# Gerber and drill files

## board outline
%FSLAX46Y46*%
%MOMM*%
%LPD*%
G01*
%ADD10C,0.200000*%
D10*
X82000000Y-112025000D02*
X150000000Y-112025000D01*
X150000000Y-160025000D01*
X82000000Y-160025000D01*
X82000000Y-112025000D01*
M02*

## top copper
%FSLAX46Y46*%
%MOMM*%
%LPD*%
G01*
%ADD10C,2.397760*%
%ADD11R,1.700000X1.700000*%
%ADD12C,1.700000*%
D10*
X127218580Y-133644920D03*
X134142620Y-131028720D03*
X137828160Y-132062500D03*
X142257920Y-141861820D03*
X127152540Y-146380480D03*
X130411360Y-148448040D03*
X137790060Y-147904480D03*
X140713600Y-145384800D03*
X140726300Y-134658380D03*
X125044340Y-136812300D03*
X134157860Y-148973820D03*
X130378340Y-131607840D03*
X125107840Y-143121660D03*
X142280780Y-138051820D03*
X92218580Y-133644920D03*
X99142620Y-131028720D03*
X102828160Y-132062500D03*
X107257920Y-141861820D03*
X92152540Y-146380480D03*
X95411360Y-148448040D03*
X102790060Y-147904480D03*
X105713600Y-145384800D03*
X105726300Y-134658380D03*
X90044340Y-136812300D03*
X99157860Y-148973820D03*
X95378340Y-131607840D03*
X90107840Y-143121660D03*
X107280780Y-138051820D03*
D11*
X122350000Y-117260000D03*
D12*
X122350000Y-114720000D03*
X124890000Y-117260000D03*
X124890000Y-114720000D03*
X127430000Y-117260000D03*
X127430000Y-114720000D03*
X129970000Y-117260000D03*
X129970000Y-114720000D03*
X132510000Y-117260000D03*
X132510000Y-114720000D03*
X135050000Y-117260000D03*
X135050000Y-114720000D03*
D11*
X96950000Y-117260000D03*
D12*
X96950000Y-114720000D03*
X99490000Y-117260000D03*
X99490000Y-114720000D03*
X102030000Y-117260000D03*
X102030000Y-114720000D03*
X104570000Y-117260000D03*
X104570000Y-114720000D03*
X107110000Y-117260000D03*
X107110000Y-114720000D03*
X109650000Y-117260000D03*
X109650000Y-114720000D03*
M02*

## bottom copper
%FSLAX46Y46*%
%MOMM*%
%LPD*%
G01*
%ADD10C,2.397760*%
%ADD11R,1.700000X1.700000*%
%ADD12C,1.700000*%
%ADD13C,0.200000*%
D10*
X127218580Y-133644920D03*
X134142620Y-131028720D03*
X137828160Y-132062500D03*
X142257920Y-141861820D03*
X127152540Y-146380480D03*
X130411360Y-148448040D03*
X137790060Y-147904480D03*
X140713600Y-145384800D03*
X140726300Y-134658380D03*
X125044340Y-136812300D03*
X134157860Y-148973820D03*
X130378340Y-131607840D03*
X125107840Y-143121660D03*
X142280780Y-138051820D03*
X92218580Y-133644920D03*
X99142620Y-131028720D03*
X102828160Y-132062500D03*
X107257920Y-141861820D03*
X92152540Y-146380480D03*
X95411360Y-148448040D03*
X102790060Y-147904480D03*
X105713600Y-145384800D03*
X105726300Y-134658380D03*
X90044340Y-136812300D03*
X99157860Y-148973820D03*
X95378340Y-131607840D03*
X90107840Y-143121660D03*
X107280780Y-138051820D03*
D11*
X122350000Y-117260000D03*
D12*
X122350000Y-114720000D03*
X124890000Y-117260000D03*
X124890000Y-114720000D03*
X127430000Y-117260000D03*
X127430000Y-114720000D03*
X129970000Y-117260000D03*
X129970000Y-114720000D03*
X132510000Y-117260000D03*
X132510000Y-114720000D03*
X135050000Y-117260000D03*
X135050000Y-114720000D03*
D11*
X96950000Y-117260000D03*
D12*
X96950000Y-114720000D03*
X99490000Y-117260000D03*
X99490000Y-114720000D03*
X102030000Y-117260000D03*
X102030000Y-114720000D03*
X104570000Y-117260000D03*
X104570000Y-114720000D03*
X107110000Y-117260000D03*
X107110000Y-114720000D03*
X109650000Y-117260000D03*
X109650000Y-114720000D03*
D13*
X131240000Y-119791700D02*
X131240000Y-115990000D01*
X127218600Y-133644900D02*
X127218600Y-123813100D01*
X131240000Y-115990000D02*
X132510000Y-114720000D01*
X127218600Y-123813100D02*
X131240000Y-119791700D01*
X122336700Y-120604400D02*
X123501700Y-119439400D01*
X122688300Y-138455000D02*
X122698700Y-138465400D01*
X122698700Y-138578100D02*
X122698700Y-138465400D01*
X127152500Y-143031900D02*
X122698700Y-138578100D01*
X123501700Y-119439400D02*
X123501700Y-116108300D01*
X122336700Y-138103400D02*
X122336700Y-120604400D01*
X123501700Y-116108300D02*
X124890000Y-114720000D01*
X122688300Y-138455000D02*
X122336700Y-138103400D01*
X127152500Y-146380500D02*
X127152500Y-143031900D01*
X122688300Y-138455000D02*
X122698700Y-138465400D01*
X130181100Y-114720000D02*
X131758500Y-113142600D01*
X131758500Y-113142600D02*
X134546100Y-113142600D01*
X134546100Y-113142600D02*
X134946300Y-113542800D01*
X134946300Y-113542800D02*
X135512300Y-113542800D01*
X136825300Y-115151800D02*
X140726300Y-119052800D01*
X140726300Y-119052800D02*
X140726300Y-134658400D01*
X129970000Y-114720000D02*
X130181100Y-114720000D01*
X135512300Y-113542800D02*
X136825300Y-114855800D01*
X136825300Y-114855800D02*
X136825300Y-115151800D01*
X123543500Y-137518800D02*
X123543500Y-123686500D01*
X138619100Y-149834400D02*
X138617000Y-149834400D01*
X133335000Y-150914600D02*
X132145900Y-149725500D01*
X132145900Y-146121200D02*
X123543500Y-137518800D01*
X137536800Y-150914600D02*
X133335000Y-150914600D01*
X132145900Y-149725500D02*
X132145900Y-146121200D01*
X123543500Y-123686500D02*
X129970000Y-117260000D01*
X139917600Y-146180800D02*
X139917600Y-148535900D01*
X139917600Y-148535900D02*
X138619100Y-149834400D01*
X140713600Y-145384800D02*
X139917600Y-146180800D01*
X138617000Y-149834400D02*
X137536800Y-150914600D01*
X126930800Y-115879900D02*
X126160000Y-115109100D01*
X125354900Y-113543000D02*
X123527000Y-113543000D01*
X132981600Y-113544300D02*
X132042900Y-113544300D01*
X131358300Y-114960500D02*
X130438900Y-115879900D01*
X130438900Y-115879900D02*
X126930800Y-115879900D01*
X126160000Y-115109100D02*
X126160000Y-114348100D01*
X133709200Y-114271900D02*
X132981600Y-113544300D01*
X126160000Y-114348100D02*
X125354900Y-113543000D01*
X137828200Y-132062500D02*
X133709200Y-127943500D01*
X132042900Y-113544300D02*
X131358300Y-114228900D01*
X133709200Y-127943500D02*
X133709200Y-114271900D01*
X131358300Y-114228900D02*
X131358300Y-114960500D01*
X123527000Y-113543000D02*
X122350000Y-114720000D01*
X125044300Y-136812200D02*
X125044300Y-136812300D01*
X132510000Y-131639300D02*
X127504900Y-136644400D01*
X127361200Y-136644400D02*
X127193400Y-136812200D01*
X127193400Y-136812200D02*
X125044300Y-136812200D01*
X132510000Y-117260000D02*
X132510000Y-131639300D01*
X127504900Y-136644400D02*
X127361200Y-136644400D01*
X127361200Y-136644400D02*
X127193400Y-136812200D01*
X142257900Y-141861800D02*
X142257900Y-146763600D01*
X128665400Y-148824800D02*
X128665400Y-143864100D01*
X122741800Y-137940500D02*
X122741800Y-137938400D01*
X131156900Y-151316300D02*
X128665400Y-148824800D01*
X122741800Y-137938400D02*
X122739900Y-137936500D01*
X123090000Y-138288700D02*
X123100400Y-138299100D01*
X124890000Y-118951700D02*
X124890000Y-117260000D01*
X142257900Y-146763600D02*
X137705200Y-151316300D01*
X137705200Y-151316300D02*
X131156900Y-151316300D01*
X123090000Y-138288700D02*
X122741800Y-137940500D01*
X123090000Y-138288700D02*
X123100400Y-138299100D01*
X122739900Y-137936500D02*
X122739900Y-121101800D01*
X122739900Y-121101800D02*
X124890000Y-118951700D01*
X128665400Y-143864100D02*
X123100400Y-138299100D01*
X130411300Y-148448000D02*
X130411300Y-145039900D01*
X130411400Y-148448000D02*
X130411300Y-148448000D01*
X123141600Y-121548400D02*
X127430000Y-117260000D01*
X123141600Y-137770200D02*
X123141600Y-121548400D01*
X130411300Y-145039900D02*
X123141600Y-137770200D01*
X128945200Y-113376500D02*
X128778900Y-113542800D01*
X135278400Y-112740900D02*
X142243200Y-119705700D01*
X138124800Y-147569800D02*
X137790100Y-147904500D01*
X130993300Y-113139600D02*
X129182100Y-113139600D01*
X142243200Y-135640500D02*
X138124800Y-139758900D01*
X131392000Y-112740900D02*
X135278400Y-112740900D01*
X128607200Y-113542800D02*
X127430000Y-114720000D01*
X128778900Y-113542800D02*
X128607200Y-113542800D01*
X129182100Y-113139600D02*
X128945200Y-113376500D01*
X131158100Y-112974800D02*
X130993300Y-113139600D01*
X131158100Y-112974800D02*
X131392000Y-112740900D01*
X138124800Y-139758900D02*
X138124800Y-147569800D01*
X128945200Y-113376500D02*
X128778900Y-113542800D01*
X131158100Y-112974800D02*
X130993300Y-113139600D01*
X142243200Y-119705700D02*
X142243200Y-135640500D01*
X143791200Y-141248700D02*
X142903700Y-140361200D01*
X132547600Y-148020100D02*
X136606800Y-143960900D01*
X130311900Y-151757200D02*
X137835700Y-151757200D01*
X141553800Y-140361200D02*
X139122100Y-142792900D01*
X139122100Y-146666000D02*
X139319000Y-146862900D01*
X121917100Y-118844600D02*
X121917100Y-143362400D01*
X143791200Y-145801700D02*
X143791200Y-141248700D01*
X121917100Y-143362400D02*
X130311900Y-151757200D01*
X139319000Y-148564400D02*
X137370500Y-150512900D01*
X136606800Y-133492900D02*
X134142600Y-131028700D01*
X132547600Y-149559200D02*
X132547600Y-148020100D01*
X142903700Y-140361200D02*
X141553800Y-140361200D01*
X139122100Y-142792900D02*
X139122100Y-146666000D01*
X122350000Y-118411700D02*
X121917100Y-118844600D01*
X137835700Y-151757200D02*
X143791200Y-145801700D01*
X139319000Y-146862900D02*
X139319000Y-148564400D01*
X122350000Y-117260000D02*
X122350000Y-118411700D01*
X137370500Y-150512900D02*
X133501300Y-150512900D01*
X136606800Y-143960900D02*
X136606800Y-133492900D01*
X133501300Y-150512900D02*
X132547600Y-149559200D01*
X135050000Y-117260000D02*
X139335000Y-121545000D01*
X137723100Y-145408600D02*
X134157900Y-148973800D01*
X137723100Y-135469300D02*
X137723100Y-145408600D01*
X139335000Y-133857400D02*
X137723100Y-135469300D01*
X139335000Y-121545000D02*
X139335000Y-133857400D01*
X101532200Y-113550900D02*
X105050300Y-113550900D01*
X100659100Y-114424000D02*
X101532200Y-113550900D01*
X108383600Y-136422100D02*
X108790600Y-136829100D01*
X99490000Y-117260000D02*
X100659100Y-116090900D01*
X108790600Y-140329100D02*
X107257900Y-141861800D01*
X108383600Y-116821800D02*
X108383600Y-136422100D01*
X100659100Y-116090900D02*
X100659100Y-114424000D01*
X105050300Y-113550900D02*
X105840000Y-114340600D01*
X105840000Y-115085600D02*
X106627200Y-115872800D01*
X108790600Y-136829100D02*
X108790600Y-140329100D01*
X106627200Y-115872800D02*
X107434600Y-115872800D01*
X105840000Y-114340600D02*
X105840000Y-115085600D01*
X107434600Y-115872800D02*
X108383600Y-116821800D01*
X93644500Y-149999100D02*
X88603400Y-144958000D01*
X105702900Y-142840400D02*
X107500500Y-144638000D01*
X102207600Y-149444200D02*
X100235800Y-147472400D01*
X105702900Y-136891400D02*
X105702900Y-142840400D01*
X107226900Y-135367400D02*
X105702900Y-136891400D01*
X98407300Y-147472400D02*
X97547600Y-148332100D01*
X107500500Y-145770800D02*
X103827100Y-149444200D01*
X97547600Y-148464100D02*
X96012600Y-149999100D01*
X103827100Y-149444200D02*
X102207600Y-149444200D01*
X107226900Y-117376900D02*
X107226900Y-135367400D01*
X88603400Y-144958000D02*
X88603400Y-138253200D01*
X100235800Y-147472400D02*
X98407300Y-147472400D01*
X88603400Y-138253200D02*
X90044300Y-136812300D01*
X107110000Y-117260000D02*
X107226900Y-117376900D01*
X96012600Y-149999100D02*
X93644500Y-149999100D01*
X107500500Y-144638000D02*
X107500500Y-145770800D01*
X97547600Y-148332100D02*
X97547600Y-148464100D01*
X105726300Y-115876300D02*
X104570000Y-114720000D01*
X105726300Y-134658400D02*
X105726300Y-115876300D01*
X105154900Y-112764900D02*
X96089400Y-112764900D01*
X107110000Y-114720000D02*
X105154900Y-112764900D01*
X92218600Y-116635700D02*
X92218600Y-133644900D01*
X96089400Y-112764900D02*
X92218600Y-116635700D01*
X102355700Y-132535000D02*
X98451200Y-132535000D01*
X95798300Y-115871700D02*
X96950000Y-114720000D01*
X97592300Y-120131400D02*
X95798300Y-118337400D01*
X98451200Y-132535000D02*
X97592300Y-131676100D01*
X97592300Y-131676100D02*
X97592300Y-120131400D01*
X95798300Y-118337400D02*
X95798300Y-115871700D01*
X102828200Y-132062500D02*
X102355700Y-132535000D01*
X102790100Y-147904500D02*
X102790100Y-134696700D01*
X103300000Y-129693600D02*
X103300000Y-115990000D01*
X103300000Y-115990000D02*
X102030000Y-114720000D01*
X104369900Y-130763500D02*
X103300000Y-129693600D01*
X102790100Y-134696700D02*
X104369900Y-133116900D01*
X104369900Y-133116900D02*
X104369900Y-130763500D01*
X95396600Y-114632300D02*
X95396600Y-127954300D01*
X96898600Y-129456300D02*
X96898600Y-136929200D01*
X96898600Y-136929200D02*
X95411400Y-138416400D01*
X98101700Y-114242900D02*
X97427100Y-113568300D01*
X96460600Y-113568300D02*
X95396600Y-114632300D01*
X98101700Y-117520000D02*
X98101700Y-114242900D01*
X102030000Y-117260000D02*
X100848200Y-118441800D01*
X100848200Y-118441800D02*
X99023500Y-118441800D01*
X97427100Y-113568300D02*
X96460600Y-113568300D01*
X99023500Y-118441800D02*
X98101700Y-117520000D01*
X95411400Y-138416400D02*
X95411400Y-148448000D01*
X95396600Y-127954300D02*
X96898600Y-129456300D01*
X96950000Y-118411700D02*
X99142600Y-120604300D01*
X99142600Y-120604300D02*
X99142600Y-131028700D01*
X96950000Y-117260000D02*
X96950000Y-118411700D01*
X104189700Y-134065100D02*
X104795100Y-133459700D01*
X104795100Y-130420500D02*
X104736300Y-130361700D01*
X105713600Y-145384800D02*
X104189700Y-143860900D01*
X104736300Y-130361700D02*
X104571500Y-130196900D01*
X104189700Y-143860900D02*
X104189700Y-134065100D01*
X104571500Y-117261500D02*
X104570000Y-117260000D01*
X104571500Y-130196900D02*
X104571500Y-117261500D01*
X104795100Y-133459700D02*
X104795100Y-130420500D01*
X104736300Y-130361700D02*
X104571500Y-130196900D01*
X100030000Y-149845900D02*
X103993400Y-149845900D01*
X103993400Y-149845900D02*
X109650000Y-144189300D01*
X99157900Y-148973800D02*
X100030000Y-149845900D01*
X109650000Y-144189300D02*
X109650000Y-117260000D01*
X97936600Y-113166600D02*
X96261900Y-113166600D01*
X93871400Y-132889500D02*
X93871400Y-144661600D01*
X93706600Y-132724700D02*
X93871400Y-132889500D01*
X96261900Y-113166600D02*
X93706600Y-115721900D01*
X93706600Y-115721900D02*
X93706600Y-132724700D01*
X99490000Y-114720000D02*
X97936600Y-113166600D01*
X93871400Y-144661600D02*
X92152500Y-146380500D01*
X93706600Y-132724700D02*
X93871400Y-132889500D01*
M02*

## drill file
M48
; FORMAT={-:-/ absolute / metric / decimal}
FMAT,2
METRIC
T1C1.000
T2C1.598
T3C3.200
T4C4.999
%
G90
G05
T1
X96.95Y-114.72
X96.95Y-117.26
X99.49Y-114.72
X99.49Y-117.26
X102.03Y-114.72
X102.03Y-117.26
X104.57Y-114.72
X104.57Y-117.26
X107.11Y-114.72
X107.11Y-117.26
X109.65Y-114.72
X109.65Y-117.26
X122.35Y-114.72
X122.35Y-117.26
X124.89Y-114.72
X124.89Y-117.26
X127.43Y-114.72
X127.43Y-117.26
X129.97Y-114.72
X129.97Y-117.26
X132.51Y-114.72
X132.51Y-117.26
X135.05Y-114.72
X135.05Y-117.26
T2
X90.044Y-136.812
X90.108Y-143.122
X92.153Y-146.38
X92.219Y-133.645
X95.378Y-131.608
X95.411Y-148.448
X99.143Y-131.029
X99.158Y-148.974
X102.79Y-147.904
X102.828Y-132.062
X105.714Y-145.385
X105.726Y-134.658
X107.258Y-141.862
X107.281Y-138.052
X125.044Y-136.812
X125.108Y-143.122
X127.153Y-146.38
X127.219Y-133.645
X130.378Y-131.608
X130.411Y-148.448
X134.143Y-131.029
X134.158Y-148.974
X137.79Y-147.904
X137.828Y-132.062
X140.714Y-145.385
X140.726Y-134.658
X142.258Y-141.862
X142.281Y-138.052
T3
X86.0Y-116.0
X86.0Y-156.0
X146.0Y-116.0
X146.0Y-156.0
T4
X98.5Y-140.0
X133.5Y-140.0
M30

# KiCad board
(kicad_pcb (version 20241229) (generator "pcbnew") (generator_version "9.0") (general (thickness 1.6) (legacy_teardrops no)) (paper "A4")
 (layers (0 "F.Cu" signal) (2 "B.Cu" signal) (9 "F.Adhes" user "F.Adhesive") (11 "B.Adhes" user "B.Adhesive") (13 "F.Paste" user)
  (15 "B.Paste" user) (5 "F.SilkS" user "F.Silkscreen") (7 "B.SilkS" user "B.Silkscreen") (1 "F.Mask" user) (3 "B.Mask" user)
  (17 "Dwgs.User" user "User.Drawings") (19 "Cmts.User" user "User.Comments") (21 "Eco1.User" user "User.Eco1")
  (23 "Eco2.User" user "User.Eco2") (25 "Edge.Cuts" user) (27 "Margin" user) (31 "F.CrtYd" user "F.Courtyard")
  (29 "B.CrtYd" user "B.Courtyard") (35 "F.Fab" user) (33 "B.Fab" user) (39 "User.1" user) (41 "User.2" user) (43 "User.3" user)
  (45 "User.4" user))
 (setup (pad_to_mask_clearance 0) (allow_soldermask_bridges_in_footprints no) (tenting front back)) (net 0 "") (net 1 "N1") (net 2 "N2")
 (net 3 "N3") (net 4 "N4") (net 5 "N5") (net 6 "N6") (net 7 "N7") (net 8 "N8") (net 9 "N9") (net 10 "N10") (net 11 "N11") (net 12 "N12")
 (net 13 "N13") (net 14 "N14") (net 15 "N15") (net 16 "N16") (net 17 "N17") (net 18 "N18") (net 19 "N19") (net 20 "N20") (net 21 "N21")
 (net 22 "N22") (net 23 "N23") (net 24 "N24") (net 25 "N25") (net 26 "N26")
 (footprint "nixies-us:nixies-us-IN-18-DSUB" (layer "F.Cu") (at 133.5 140 180)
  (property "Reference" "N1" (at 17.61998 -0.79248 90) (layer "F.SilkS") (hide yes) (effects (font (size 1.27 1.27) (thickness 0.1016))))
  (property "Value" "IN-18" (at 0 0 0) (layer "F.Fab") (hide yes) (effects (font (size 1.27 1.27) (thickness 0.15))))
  (pad "" np_thru_hole circle (at 0 0 180) (size 4.99872 4.99872) (drill 4.99872) (layers "*.Cu" "*.Mask"))
  (pad "0" thru_hole circle (at 6.28142 6.35508 180) (size 2.39776 2.39776) (drill 1.59766) (layers "*.Cu" "*.Mask")
   (remove_unused_layers no) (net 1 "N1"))
  (pad "1" thru_hole circle (at -0.64262 8.97128 180) (size 2.39776 2.39776) (drill 1.59766) (layers "*.Cu" "*.Mask")
   (remove_unused_layers no) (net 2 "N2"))
  (pad "2" thru_hole circle (at -4.32816 7.9375 180) (size 2.39776 2.39776) (drill 1.59766) (layers "*.Cu" "*.Mask")
   (remove_unused_layers no) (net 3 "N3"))
  (pad "3" thru_hole circle (at -8.75792 -1.86182 180) (size 2.39776 2.39776) (drill 1.59766) (layers "*.Cu" "*.Mask")
   (remove_unused_layers no) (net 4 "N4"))
  (pad "4" thru_hole circle (at 6.34746 -6.38048 180) (size 2.39776 2.39776) (drill 1.59766) (layers "*.Cu" "*.Mask")
   (remove_unused_layers no) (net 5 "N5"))
  (pad "5" thru_hole circle (at 3.08864 -8.44804 180) (size 2.39776 2.39776) (drill 1.59766) (layers "*.Cu" "*.Mask")
   (remove_unused_layers no) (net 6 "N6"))
  (pad "6" thru_hole circle (at -4.29006 -7.90448 180) (size 2.39776 2.39776) (drill 1.59766) (layers "*.Cu" "*.Mask")
   (remove_unused_layers no) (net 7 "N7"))
  (pad "7" thru_hole circle (at -7.2136 -5.3848 180) (size 2.39776 2.39776) (drill 1.59766) (layers "*.Cu" "*.Mask")
   (remove_unused_layers no) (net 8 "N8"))
  (pad "8" thru_hole circle (at -7.2263 5.34162 180) (size 2.39776 2.39776) (drill 1.59766) (layers "*.Cu" "*.Mask")
   (remove_unused_layers no) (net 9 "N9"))
  (pad "9" thru_hole circle (at 8.45566 3.1877 180) (size 2.39776 2.39776) (drill 1.59766) (layers "*.Cu" "*.Mask")
   (remove_unused_layers no) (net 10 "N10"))
  (pad "A" thru_hole circle (at -0.65786 -8.97382 180) (size 2.39776 2.39776) (drill 1.59766) (layers "*.Cu" "*.Mask")
   (remove_unused_layers no) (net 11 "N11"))
  (pad "A2" thru_hole circle (at 3.12166 8.39216 180) (size 2.39776 2.39776) (drill 1.59766) (layers "*.Cu" "*.Mask")
   (remove_unused_layers no) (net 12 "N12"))
  (pad "N/C" thru_hole circle (at 8.39216 -3.12166 180) (size 2.39776 2.39776) (drill 1.59766) (layers "*.Cu" "*.Mask")
   (remove_unused_layers no))
  (pad "N/C2" thru_hole circle (at -8.78078 1.94818 180) (size 2.39776 2.39776) (drill 1.59766) (layers "*.Cu" "*.Mask")
   (remove_unused_layers no)))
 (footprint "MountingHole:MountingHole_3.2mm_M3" (layer "F.Cu") (at 86 116)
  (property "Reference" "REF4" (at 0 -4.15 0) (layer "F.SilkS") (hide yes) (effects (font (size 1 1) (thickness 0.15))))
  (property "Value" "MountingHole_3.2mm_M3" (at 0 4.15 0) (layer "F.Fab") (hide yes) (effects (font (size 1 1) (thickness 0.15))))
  (pad "" np_thru_hole circle (at 0 0) (size 3.2 3.2) (drill 3.2) (layers "*.Cu" "*.Mask")))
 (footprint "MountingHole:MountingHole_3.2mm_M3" (layer "F.Cu") (at 146 116)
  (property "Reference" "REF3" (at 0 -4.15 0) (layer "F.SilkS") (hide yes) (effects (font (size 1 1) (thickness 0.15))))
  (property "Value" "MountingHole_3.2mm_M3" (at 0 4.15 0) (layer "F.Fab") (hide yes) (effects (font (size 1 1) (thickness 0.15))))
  (pad "" np_thru_hole circle (at 0 0) (size 3.2 3.2) (drill 3.2) (layers "*.Cu" "*.Mask")))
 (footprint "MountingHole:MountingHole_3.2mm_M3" (layer "F.Cu") (at 146 156)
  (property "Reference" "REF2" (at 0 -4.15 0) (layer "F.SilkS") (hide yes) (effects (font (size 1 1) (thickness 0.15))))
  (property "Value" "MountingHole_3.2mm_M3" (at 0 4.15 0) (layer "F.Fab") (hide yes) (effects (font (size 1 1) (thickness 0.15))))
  (pad "" np_thru_hole circle (at 0 0) (size 3.2 3.2) (drill 3.2) (layers "*.Cu" "*.Mask")))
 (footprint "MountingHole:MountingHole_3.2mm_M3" (layer "F.Cu") (at 86 156)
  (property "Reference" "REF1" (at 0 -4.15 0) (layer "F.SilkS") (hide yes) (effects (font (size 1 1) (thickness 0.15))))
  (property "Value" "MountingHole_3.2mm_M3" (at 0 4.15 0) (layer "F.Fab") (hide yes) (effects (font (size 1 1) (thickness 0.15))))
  (pad "" np_thru_hole circle (at 0 0) (size 3.2 3.2) (drill 3.2) (layers "*.Cu" "*.Mask")))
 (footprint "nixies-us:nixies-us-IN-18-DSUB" (layer "F.Cu") (at 98.5 140 180)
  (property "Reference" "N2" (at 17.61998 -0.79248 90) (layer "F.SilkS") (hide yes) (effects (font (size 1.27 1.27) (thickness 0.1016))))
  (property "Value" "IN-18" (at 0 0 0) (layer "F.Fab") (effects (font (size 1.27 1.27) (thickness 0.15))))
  (pad "" np_thru_hole circle (at 0 0 180) (size 4.99872 4.99872) (drill 4.99872) (layers "*.Cu" "*.Mask"))
  (pad "0" thru_hole circle (at 6.28142 6.35508 180) (size 2.39776 2.39776) (drill 1.59766) (layers "*.Cu" "*.Mask")
   (remove_unused_layers no) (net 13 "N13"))
  (pad "1" thru_hole circle (at -0.64262 8.97128 180) (size 2.39776 2.39776) (drill 1.59766) (layers "*.Cu" "*.Mask")
   (remove_unused_layers no) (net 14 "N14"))
  (pad "2" thru_hole circle (at -4.32816 7.9375 180) (size 2.39776 2.39776) (drill 1.59766) (layers "*.Cu" "*.Mask")
   (remove_unused_layers no) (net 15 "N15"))
  (pad "3" thru_hole circle (at -8.75792 -1.86182 180) (size 2.39776 2.39776) (drill 1.59766) (layers "*.Cu" "*.Mask")
   (remove_unused_layers no) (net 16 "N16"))
  (pad "4" thru_hole circle (at 6.34746 -6.38048 180) (size 2.39776 2.39776) (drill 1.59766) (layers "*.Cu" "*.Mask")
   (remove_unused_layers no) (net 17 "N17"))
  (pad "5" thru_hole circle (at 3.08864 -8.44804 180) (size 2.39776 2.39776) (drill 1.59766) (layers "*.Cu" "*.Mask")
   (remove_unused_layers no) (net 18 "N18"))
  (pad "6" thru_hole circle (at -4.29006 -7.90448 180) (size 2.39776 2.39776) (drill 1.59766) (layers "*.Cu" "*.Mask")
   (remove_unused_layers no) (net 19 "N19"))
  (pad "7" thru_hole circle (at -7.2136 -5.3848 180) (size 2.39776 2.39776) (drill 1.59766) (layers "*.Cu" "*.Mask")
   (remove_unused_layers no) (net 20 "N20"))
  (pad "8" thru_hole circle (at -7.2263 5.34162 180) (size 2.39776 2.39776) (drill 1.59766) (layers "*.Cu" "*.Mask")
   (remove_unused_layers no) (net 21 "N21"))
  (pad "9" thru_hole circle (at 8.45566 3.1877 180) (size 2.39776 2.39776) (drill 1.59766) (layers "*.Cu" "*.Mask")
   (remove_unused_layers no) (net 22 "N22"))
  (pad "A" thru_hole circle (at -0.65786 -8.97382 180) (size 2.39776 2.39776) (drill 1.59766) (layers "*.Cu" "*.Mask")
   (remove_unused_layers no) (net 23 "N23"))
  (pad "A2" thru_hole circle (at 3.12166 8.39216 180) (size 2.39776 2.39776) (drill 1.59766) (layers "*.Cu" "*.Mask")
   (remove_unused_layers no) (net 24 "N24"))
  (pad "N/C" thru_hole circle (at 8.39216 -3.12166 180) (size 2.39776 2.39776) (drill 1.59766) (layers "*.Cu" "*.Mask")
   (remove_unused_layers no))
  (pad "N/C2" thru_hole circle (at -8.78078 1.94818 180) (size 2.39776 2.39776) (drill 1.59766) (layers "*.Cu" "*.Mask")
   (remove_unused_layers no)))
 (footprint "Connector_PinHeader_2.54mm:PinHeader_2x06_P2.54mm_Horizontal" (layer "F.Cu") (at 122.35 117.26 90)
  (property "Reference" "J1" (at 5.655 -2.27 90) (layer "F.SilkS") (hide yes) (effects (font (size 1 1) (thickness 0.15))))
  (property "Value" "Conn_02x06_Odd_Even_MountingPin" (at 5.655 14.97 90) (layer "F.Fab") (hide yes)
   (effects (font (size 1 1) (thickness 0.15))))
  (pad "1" thru_hole rect (at 0 0 90) (size 1.7 1.7) (drill 1) (layers "*.Cu" "*.Mask") (remove_unused_layers no) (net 2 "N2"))
  (pad "2" thru_hole circle (at 2.54 0 90) (size 1.7 1.7) (drill 1) (layers "*.Cu" "*.Mask") (remove_unused_layers no) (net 3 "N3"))
  (pad "3" thru_hole circle (at 0 2.54 90) (size 1.7 1.7) (drill 1) (layers "*.Cu" "*.Mask") (remove_unused_layers no) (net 4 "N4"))
  (pad "4" thru_hole circle (at 2.54 2.54 90) (size 1.7 1.7) (drill 1) (layers "*.Cu" "*.Mask") (remove_unused_layers no) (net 5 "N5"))
  (pad "5" thru_hole circle (at 0 5.08 90) (size 1.7 1.7) (drill 1) (layers "*.Cu" "*.Mask") (remove_unused_layers no) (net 6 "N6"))
  (pad "6" thru_hole circle (at 2.54 5.08 90) (size 1.7 1.7) (drill 1) (layers "*.Cu" "*.Mask") (remove_unused_layers no) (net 7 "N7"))
  (pad "7" thru_hole circle (at 0 7.62 90) (size 1.7 1.7) (drill 1) (layers "*.Cu" "*.Mask") (remove_unused_layers no) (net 8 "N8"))
  (pad "8" thru_hole circle (at 2.54 7.62 90) (size 1.7 1.7) (drill 1) (layers "*.Cu" "*.Mask") (remove_unused_layers no) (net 9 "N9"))
  (pad "9" thru_hole circle (at 0 10.16 90) (size 1.7 1.7) (drill 1) (layers "*.Cu" "*.Mask") (remove_unused_layers no) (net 10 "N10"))
  (pad "10" thru_hole circle (at 2.54 10.16 90) (size 1.7 1.7) (drill 1) (layers "*.Cu" "*.Mask") (remove_unused_layers no) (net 1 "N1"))
  (pad "11" thru_hole circle (at 0 12.7 90) (size 1.7 1.7) (drill 1) (layers "*.Cu" "*.Mask") (remove_unused_layers no) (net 11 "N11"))
  (pad "12" thru_hole circle (at 2.54 12.7 90) (size 1.7 1.7) (drill 1) (layers "*.Cu" "*.Mask") (remove_unused_layers no) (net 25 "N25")))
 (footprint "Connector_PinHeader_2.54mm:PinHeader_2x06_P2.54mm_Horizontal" (layer "F.Cu") (at 96.95 117.26 90)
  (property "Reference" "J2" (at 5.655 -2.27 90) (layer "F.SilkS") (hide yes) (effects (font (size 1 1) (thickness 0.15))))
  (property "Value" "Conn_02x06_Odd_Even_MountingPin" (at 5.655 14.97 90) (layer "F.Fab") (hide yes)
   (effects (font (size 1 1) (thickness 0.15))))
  (pad "1" thru_hole rect (at 0 0 90) (size 1.7 1.7) (drill 1) (layers "*.Cu" "*.Mask") (remove_unused_layers no) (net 14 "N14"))
  (pad "2" thru_hole circle (at 2.54 0 90) (size 1.7 1.7) (drill 1) (layers "*.Cu" "*.Mask") (remove_unused_layers no) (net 15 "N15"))
  (pad "3" thru_hole circle (at 0 2.54 90) (size 1.7 1.7) (drill 1) (layers "*.Cu" "*.Mask") (remove_unused_layers no) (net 16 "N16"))
  (pad "4" thru_hole circle (at 2.54 2.54 90) (size 1.7 1.7) (drill 1) (layers "*.Cu" "*.Mask") (remove_unused_layers no) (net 17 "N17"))
  (pad "5" thru_hole circle (at 0 5.08 90) (size 1.7 1.7) (drill 1) (layers "*.Cu" "*.Mask") (remove_unused_layers no) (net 18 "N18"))
  (pad "6" thru_hole circle (at 2.54 5.08 90) (size 1.7 1.7) (drill 1) (layers "*.Cu" "*.Mask") (remove_unused_layers no) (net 19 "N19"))
  (pad "7" thru_hole circle (at 0 7.62 90) (size 1.7 1.7) (drill 1) (layers "*.Cu" "*.Mask") (remove_unused_layers no) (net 20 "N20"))
  (pad "8" thru_hole circle (at 2.54 7.62 90) (size 1.7 1.7) (drill 1) (layers "*.Cu" "*.Mask") (remove_unused_layers no) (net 21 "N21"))
  (pad "9" thru_hole circle (at 0 10.16 90) (size 1.7 1.7) (drill 1) (layers "*.Cu" "*.Mask") (remove_unused_layers no) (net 22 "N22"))
  (pad "10" thru_hole circle (at 2.54 10.16 90) (size 1.7 1.7) (drill 1) (layers "*.Cu" "*.Mask") (remove_unused_layers no) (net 13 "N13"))
  (pad "11" thru_hole circle (at 0 12.7 90) (size 1.7 1.7) (drill 1) (layers "*.Cu" "*.Mask") (remove_unused_layers no) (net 23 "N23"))
  (pad "12" thru_hole circle (at 2.54 12.7 90) (size 1.7 1.7) (drill 1) (layers "*.Cu" "*.Mask") (remove_unused_layers no) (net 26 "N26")))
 (gr_rect (start 82 112.025) (end 150 160.025) (stroke (width 0.2) (type solid)) (fill no) (layer "Edge.Cuts"))
 (segment (start 131.24 119.7917) (end 131.24 115.99) (width 0.2) (layer "B.Cu") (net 1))
 (segment (start 127.2186 133.6449) (end 127.2186 123.8131) (width 0.2) (layer "B.Cu") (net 1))
 (segment (start 131.24 115.99) (end 132.51 114.72) (width 0.2) (layer "B.Cu") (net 1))
 (segment (start 127.2186 123.8131) (end 131.24 119.7917) (width 0.2) (layer "B.Cu") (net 1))
 (segment (start 122.3367 120.6044) (end 123.5017 119.4394) (width 0.2) (layer "B.Cu") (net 5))
 (segment (start 122.6883 138.455) (end 122.6987 138.4654) (width 0.2) (layer "B.Cu") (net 5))
 (segment (start 122.6987 138.5781) (end 122.6987 138.4654) (width 0.2) (layer "B.Cu") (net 5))
 (segment (start 127.1525 143.0319) (end 122.6987 138.5781) (width 0.2) (layer "B.Cu") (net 5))
 (segment (start 123.5017 119.4394) (end 123.5017 116.1083) (width 0.2) (layer "B.Cu") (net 5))
 (segment (start 122.3367 138.1034) (end 122.3367 120.6044) (width 0.2) (layer "B.Cu") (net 5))
 (segment (start 123.5017 116.1083) (end 124.89 114.72) (width 0.2) (layer "B.Cu") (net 5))
 (segment (start 122.6883 138.455) (end 122.3367 138.1034) (width 0.2) (layer "B.Cu") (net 5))
 (segment (start 127.1525 146.3805) (end 127.1525 143.0319) (width 0.2) (layer "B.Cu") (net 5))
 (segment (start 122.6883 138.455) (end 122.6987 138.4654) (width 0.2) (layer "B.Cu") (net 5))
 (segment (start 130.1811 114.72) (end 131.7585 113.1426) (width 0.2) (layer "B.Cu") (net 9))
 (segment (start 131.7585 113.1426) (end 134.5461 113.1426) (width 0.2) (layer "B.Cu") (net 9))
 (segment (start 134.5461 113.1426) (end 134.9463 113.5428) (width 0.2) (layer "B.Cu") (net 9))
 (segment (start 134.9463 113.5428) (end 135.5123 113.5428) (width 0.2) (layer "B.Cu") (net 9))
 (segment (start 136.8253 115.1518) (end 140.7263 119.0528) (width 0.2) (layer "B.Cu") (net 9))
 (segment (start 140.7263 119.0528) (end 140.7263 134.6584) (width 0.2) (layer "B.Cu") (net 9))
 (segment (start 129.97 114.72) (end 130.1811 114.72) (width 0.2) (layer "B.Cu") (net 9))
 (segment (start 135.5123 113.5428) (end 136.8253 114.8558) (width 0.2) (layer "B.Cu") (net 9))
 (segment (start 136.8253 114.8558) (end 136.8253 115.1518) (width 0.2) (layer "B.Cu") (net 9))
 (segment (start 123.5435 137.5188) (end 123.5435 123.6865) (width 0.2) (layer "B.Cu") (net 8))
 (segment (start 138.6191 149.8344) (end 138.617 149.8344) (width 0.2) (layer "B.Cu") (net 8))
 (segment (start 133.335 150.9146) (end 132.1459 149.7255) (width 0.2) (layer "B.Cu") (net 8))
 (segment (start 132.1459 146.1212) (end 123.5435 137.5188) (width 0.2) (layer "B.Cu") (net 8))
 (segment (start 137.5368 150.9146) (end 133.335 150.9146) (width 0.2) (layer "B.Cu") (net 8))
 (segment (start 132.1459 149.7255) (end 132.1459 146.1212) (width 0.2) (layer "B.Cu") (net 8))
 (segment (start 123.5435 123.6865) (end 129.97 117.26) (width 0.2) (layer "B.Cu") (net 8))
 (segment (start 139.9176 146.1808) (end 139.9176 148.5359) (width 0.2) (layer "B.Cu") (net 8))
 (segment (start 139.9176 148.5359) (end 138.6191 149.8344) (width 0.2) (layer "B.Cu") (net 8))
 (segment (start 140.7136 145.3848) (end 139.9176 146.1808) (width 0.2) (layer "B.Cu") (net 8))
 (segment (start 138.617 149.8344) (end 137.5368 150.9146) (width 0.2) (layer "B.Cu") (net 8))
 (segment (start 126.9308 115.8799) (end 126.16 115.1091) (width 0.2) (layer "B.Cu") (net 3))
 (segment (start 125.3549 113.543) (end 123.527 113.543) (width 0.2) (layer "B.Cu") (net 3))
 (segment (start 132.9816 113.5443) (end 132.0429 113.5443) (width 0.2) (layer "B.Cu") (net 3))
 (segment (start 131.3583 114.9605) (end 130.4389 115.8799) (width 0.2) (layer "B.Cu") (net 3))
 (segment (start 130.4389 115.8799) (end 126.9308 115.8799) (width 0.2) (layer "B.Cu") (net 3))
 (segment (start 126.16 115.1091) (end 126.16 114.3481) (width 0.2) (layer "B.Cu") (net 3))
 (segment (start 133.7092 114.2719) (end 132.9816 113.5443) (width 0.2) (layer "B.Cu") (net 3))
 (segment (start 126.16 114.3481) (end 125.3549 113.543) (width 0.2) (layer "B.Cu") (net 3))
 (segment (start 137.8282 132.0625) (end 133.7092 127.9435) (width 0.2) (layer "B.Cu") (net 3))
 (segment (start 132.0429 113.5443) (end 131.3583 114.2289) (width 0.2) (layer "B.Cu") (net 3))
 (segment (start 133.7092 127.9435) (end 133.7092 114.2719) (width 0.2) (layer "B.Cu") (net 3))
 (segment (start 131.3583 114.2289) (end 131.3583 114.9605) (width 0.2) (layer "B.Cu") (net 3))
 (segment (start 123.527 113.543) (end 122.35 114.72) (width 0.2) (layer "B.Cu") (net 3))
 (segment (start 125.0443 136.8122) (end 125.0443 136.8123) (width 0.2) (layer "B.Cu") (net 10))
 (segment (start 132.51 131.6393) (end 127.5049 136.6444) (width 0.2) (layer "B.Cu") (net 10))
 (segment (start 127.3612 136.6444) (end 127.1934 136.8122) (width 0.2) (layer "B.Cu") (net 10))
 (segment (start 127.1934 136.8122) (end 125.0443 136.8122) (width 0.2) (layer "B.Cu") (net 10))
 (segment (start 132.51 117.26) (end 132.51 131.6393) (width 0.2) (layer "B.Cu") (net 10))
 (segment (start 127.5049 136.6444) (end 127.3612 136.6444) (width 0.2) (layer "B.Cu") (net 10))
 (segment (start 127.3612 136.6444) (end 127.1934 136.8122) (width 0.2) (layer "B.Cu") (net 10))
 (segment (start 142.2579 141.8618) (end 142.2579 146.7636) (width 0.2) (layer "B.Cu") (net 4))
 (segment (start 128.6654 148.8248) (end 128.6654 143.8641) (width 0.2) (layer "B.Cu") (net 4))
 (segment (start 122.7418 137.9405) (end 122.7418 137.9384) (width 0.2) (layer "B.Cu") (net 4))
 (segment (start 131.1569 151.3163) (end 128.6654 148.8248) (width 0.2) (layer "B.Cu") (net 4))
 (segment (start 122.7418 137.9384) (end 122.7399 137.9365) (width 0.2) (layer "B.Cu") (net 4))
 (segment (start 123.09 138.2887) (end 123.1004 138.2991) (width 0.2) (layer "B.Cu") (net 4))
 (segment (start 124.89 118.9517) (end 124.89 117.26) (width 0.2) (layer "B.Cu") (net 4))
 (segment (start 142.2579 146.7636) (end 137.7052 151.3163) (width 0.2) (layer "B.Cu") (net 4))
 (segment (start 137.7052 151.3163) (end 131.1569 151.3163) (width 0.2) (layer "B.Cu") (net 4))
 (segment (start 123.09 138.2887) (end 122.7418 137.9405) (width 0.2) (layer "B.Cu") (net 4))
 (segment (start 123.09 138.2887) (end 123.1004 138.2991) (width 0.2) (layer "B.Cu") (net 4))
 (segment (start 122.7399 137.9365) (end 122.7399 121.1018) (width 0.2) (layer "B.Cu") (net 4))
 (segment (start 122.7399 121.1018) (end 124.89 118.9517) (width 0.2) (layer "B.Cu") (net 4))
 (segment (start 128.6654 143.8641) (end 123.1004 138.2991) (width 0.2) (layer "B.Cu") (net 4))
 (segment (start 130.4113 148.448) (end 130.4113 145.0399) (width 0.2) (layer "B.Cu") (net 6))
 (segment (start 130.4114 148.448) (end 130.4113 148.448) (width 0.2) (layer "B.Cu") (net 6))
 (segment (start 123.1416 121.5484) (end 127.43 117.26) (width 0.2) (layer "B.Cu") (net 6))
 (segment (start 123.1416 137.7702) (end 123.1416 121.5484) (width 0.2) (layer "B.Cu") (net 6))
 (segment (start 130.4113 145.0399) (end 123.1416 137.7702) (width 0.2) (layer "B.Cu") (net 6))
 (segment (start 128.9452 113.3765) (end 128.7789 113.5428) (width 0.2) (layer "B.Cu") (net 7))
 (segment (start 135.2784 112.7409) (end 142.2432 119.7057) (width 0.2) (layer "B.Cu") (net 7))
 (segment (start 138.1248 147.5698) (end 137.7901 147.9045) (width 0.2) (layer "B.Cu") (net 7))
 (segment (start 130.9933 113.1396) (end 129.1821 113.1396) (width 0.2) (layer "B.Cu") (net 7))
 (segment (start 142.2432 135.6405) (end 138.1248 139.7589) (width 0.2) (layer "B.Cu") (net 7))
 (segment (start 131.392 112.7409) (end 135.2784 112.7409) (width 0.2) (layer "B.Cu") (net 7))
 (segment (start 128.6072 113.5428) (end 127.43 114.72) (width 0.2) (layer "B.Cu") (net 7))
 (segment (start 128.7789 113.5428) (end 128.6072 113.5428) (width 0.2) (layer "B.Cu") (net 7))
 (segment (start 129.1821 113.1396) (end 128.9452 113.3765) (width 0.2) (layer "B.Cu") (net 7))
 (segment (start 131.1581 112.9748) (end 130.9933 113.1396) (width 0.2) (layer "B.Cu") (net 7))
 (segment (start 131.1581 112.9748) (end 131.392 112.7409) (width 0.2) (layer "B.Cu") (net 7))
 (segment (start 138.1248 139.7589) (end 138.1248 147.5698) (width 0.2) (layer "B.Cu") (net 7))
 (segment (start 128.9452 113.3765) (end 128.7789 113.5428) (width 0.2) (layer "B.Cu") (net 7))
 (segment (start 131.1581 112.9748) (end 130.9933 113.1396) (width 0.2) (layer "B.Cu") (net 7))
 (segment (start 142.2432 119.7057) (end 142.2432 135.6405) (width 0.2) (layer "B.Cu") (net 7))
 (segment (start 143.7912 141.2487) (end 142.9037 140.3612) (width 0.2) (layer "B.Cu") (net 2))
 (segment (start 132.5476 148.0201) (end 136.6068 143.9609) (width 0.2) (layer "B.Cu") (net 2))
 (segment (start 130.3119 151.7572) (end 137.8357 151.7572) (width 0.2) (layer "B.Cu") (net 2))
 (segment (start 141.5538 140.3612) (end 139.1221 142.7929) (width 0.2) (layer "B.Cu") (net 2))
 (segment (start 139.1221 146.666) (end 139.319 146.8629) (width 0.2) (layer "B.Cu") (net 2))
 (segment (start 121.9171 118.8446) (end 121.9171 143.3624) (width 0.2) (layer "B.Cu") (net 2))
 (segment (start 143.7912 145.8017) (end 143.7912 141.2487) (width 0.2) (layer "B.Cu") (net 2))
 (segment (start 121.9171 143.3624) (end 130.3119 151.7572) (width 0.2) (layer "B.Cu") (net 2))
 (segment (start 139.319 148.5644) (end 137.3705 150.5129) (width 0.2) (layer "B.Cu") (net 2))
 (segment (start 136.6068 133.4929) (end 134.1426 131.0287) (width 0.2) (layer "B.Cu") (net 2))
 (segment (start 132.5476 149.5592) (end 132.5476 148.0201) (width 0.2) (layer "B.Cu") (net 2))
 (segment (start 142.9037 140.3612) (end 141.5538 140.3612) (width 0.2) (layer "B.Cu") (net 2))
 (segment (start 139.1221 142.7929) (end 139.1221 146.666) (width 0.2) (layer "B.Cu") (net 2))
 (segment (start 122.35 118.4117) (end 121.9171 118.8446) (width 0.2) (layer "B.Cu") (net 2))
 (segment (start 137.8357 151.7572) (end 143.7912 145.8017) (width 0.2) (layer "B.Cu") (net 2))
 (segment (start 139.319 146.8629) (end 139.319 148.5644) (width 0.2) (layer "B.Cu") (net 2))
 (segment (start 122.35 117.26) (end 122.35 118.4117) (width 0.2) (layer "B.Cu") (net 2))
 (segment (start 137.3705 150.5129) (end 133.5013 150.5129) (width 0.2) (layer "B.Cu") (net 2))
 (segment (start 136.6068 143.9609) (end 136.6068 133.4929) (width 0.2) (layer "B.Cu") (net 2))
 (segment (start 133.5013 150.5129) (end 132.5476 149.5592) (width 0.2) (layer "B.Cu") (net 2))
 (segment (start 135.05 117.26) (end 139.335 121.545) (width 0.2) (layer "B.Cu") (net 11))
 (segment (start 137.7231 145.4086) (end 134.1579 148.9738) (width 0.2) (layer "B.Cu") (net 11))
 (segment (start 137.7231 135.4693) (end 137.7231 145.4086) (width 0.2) (layer "B.Cu") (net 11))
 (segment (start 139.335 133.8574) (end 137.7231 135.4693) (width 0.2) (layer "B.Cu") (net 11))
 (segment (start 139.335 121.545) (end 139.335 133.8574) (width 0.2) (layer "B.Cu") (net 11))
 (segment (start 101.5322 113.5509) (end 105.0503 113.5509) (width 0.2) (layer "B.Cu") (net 16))
 (segment (start 100.6591 114.424) (end 101.5322 113.5509) (width 0.2) (layer "B.Cu") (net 16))
 (segment (start 108.3836 136.4221) (end 108.7906 136.8291) (width 0.2) (layer "B.Cu") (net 16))
 (segment (start 99.49 117.26) (end 100.6591 116.0909) (width 0.2) (layer "B.Cu") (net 16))
 (segment (start 108.7906 140.3291) (end 107.2579 141.8618) (width 0.2) (layer "B.Cu") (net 16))
 (segment (start 108.3836 116.8218) (end 108.3836 136.4221) (width 0.2) (layer "B.Cu") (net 16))
 (segment (start 100.6591 116.0909) (end 100.6591 114.424) (width 0.2) (layer "B.Cu") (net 16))
 (segment (start 105.0503 113.5509) (end 105.84 114.3406) (width 0.2) (layer "B.Cu") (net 16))
 (segment (start 105.84 115.0856) (end 106.6272 115.8728) (width 0.2) (layer "B.Cu") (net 16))
 (segment (start 108.7906 136.8291) (end 108.7906 140.3291) (width 0.2) (layer "B.Cu") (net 16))
 (segment (start 106.6272 115.8728) (end 107.4346 115.8728) (width 0.2) (layer "B.Cu") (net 16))
 (segment (start 105.84 114.3406) (end 105.84 115.0856) (width 0.2) (layer "B.Cu") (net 16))
 (segment (start 107.4346 115.8728) (end 108.3836 116.8218) (width 0.2) (layer "B.Cu") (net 16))
 (segment (start 93.6445 149.9991) (end 88.6034 144.958) (width 0.2) (layer "B.Cu") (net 22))
 (segment (start 105.7029 142.8404) (end 107.5005 144.638) (width 0.2) (layer "B.Cu") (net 22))
 (segment (start 102.2076 149.4442) (end 100.2358 147.4724) (width 0.2) (layer "B.Cu") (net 22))
 (segment (start 105.7029 136.8914) (end 105.7029 142.8404) (width 0.2) (layer "B.Cu") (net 22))
 (segment (start 107.2269 135.3674) (end 105.7029 136.8914) (width 0.2) (layer "B.Cu") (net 22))
 (segment (start 98.4073 147.4724) (end 97.5476 148.3321) (width 0.2) (layer "B.Cu") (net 22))
 (segment (start 107.5005 145.7708) (end 103.8271 149.4442) (width 0.2) (layer "B.Cu") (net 22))
 (segment (start 97.5476 148.4641) (end 96.0126 149.9991) (width 0.2) (layer "B.Cu") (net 22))
 (segment (start 103.8271 149.4442) (end 102.2076 149.4442) (width 0.2) (layer "B.Cu") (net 22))
 (segment (start 107.2269 117.3769) (end 107.2269 135.3674) (width 0.2) (layer "B.Cu") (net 22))
 (segment (start 88.6034 144.958) (end 88.6034 138.2532) (width 0.2) (layer "B.Cu") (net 22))
 (segment (start 100.2358 147.4724) (end 98.4073 147.4724) (width 0.2) (layer "B.Cu") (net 22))
 (segment (start 88.6034 138.2532) (end 90.0443 136.8123) (width 0.2) (layer "B.Cu") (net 22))
 (segment (start 107.11 117.26) (end 107.2269 117.3769) (width 0.2) (layer "B.Cu") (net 22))
 (segment (start 96.0126 149.9991) (end 93.6445 149.9991) (width 0.2) (layer "B.Cu") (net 22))
 (segment (start 107.5005 144.638) (end 107.5005 145.7708) (width 0.2) (layer "B.Cu") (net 22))
 (segment (start 97.5476 148.3321) (end 97.5476 148.4641) (width 0.2) (layer "B.Cu") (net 22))
 (segment (start 105.7263 115.8763) (end 104.57 114.72) (width 0.2) (layer "B.Cu") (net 21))
 (segment (start 105.7263 134.6584) (end 105.7263 115.8763) (width 0.2) (layer "B.Cu") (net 21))
 (segment (start 105.1549 112.7649) (end 96.0894 112.7649) (width 0.2) (layer "B.Cu") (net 13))
 (segment (start 107.11 114.72) (end 105.1549 112.7649) (width 0.2) (layer "B.Cu") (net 13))
 (segment (start 92.2186 116.6357) (end 92.2186 133.6449) (width 0.2) (layer "B.Cu") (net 13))
 (segment (start 96.0894 112.7649) (end 92.2186 116.6357) (width 0.2) (layer "B.Cu") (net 13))
 (segment (start 102.3557 132.535) (end 98.4512 132.535) (width 0.2) (layer "B.Cu") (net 15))
 (segment (start 95.7983 115.8717) (end 96.95 114.72) (width 0.2) (layer "B.Cu") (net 15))
 (segment (start 97.5923 120.1314) (end 95.7983 118.3374) (width 0.2) (layer "B.Cu") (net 15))
 (segment (start 98.4512 132.535) (end 97.5923 131.6761) (width 0.2) (layer "B.Cu") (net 15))
 (segment (start 97.5923 131.6761) (end 97.5923 120.1314) (width 0.2) (layer "B.Cu") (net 15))
 (segment (start 95.7983 118.3374) (end 95.7983 115.8717) (width 0.2) (layer "B.Cu") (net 15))
 (segment (start 102.8282 132.0625) (end 102.3557 132.535) (width 0.2) (layer "B.Cu") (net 15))
 (segment (start 102.7901 147.9045) (end 102.7901 134.6967) (width 0.2) (layer "B.Cu") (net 19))
 (segment (start 103.3 129.6936) (end 103.3 115.99) (width 0.2) (layer "B.Cu") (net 19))
 (segment (start 103.3 115.99) (end 102.03 114.72) (width 0.2) (layer "B.Cu") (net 19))
 (segment (start 104.3699 130.7635) (end 103.3 129.6936) (width 0.2) (layer "B.Cu") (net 19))
 (segment (start 102.7901 134.6967) (end 104.3699 133.1169) (width 0.2) (layer "B.Cu") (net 19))
 (segment (start 104.3699 133.1169) (end 104.3699 130.7635) (width 0.2) (layer "B.Cu") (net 19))
 (segment (start 95.3966 114.6323) (end 95.3966 127.9543) (width 0.2) (layer "B.Cu") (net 18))
 (segment (start 96.8986 129.4563) (end 96.8986 136.9292) (width 0.2) (layer "B.Cu") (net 18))
 (segment (start 96.8986 136.9292) (end 95.4114 138.4164) (width 0.2) (layer "B.Cu") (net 18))
 (segment (start 98.1017 114.2429) (end 97.4271 113.5683) (width 0.2) (layer "B.Cu") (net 18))
 (segment (start 96.4606 113.5683) (end 95.3966 114.6323) (width 0.2) (layer "B.Cu") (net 18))
 (segment (start 98.1017 117.52) (end 98.1017 114.2429) (width 0.2) (layer "B.Cu") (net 18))
 (segment (start 102.03 117.26) (end 100.8482 118.4418) (width 0.2) (layer "B.Cu") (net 18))
 (segment (start 100.8482 118.4418) (end 99.0235 118.4418) (width 0.2) (layer "B.Cu") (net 18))
 (segment (start 97.4271 113.5683) (end 96.4606 113.5683) (width 0.2) (layer "B.Cu") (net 18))
 (segment (start 99.0235 118.4418) (end 98.1017 117.52) (width 0.2) (layer "B.Cu") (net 18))
 (segment (start 95.4114 138.4164) (end 95.4114 148.448) (width 0.2) (layer "B.Cu") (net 18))
 (segment (start 95.3966 127.9543) (end 96.8986 129.4563) (width 0.2) (layer "B.Cu") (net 18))
 (segment (start 96.95 118.4117) (end 99.1426 120.6043) (width 0.2) (layer "B.Cu") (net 14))
 (segment (start 99.1426 120.6043) (end 99.1426 131.0287) (width 0.2) (layer "B.Cu") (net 14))
 (segment (start 96.95 117.26) (end 96.95 118.4117) (width 0.2) (layer "B.Cu") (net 14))
 (segment (start 104.1897 134.0651) (end 104.7951 133.4597) (width 0.2) (layer "B.Cu") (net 20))
 (segment (start 104.7951 130.4205) (end 104.7363 130.3617) (width 0.2) (layer "B.Cu") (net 20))
 (segment (start 105.7136 145.3848) (end 104.1897 143.8609) (width 0.2) (layer "B.Cu") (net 20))
 (segment (start 104.7363 130.3617) (end 104.5715 130.1969) (width 0.2) (layer "B.Cu") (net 20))
 (segment (start 104.1897 143.8609) (end 104.1897 134.0651) (width 0.2) (layer "B.Cu") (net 20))
 (segment (start 104.5715 117.2615) (end 104.57 117.26) (width 0.2) (layer "B.Cu") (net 20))
 (segment (start 104.5715 130.1969) (end 104.5715 117.2615) (width 0.2) (layer "B.Cu") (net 20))
 (segment (start 104.7951 133.4597) (end 104.7951 130.4205) (width 0.2) (layer "B.Cu") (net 20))
 (segment (start 104.7363 130.3617) (end 104.5715 130.1969) (width 0.2) (layer "B.Cu") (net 20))
 (segment (start 100.03 149.8459) (end 103.9934 149.8459) (width 0.2) (layer "B.Cu") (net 23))
 (segment (start 103.9934 149.8459) (end 109.65 144.1893) (width 0.2) (layer "B.Cu") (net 23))
 (segment (start 99.1579 148.9738) (end 100.03 149.8459) (width 0.2) (layer "B.Cu") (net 23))
 (segment (start 109.65 144.1893) (end 109.65 117.26) (width 0.2) (layer "B.Cu") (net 23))
 (segment (start 97.9366 113.1666) (end 96.2619 113.1666) (width 0.2) (layer "B.Cu") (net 17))
 (segment (start 93.8714 132.8895) (end 93.8714 144.6616) (width 0.2) (layer "B.Cu") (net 17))
 (segment (start 93.7066 132.7247) (end 93.8714 132.8895) (width 0.2) (layer "B.Cu") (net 17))
 (segment (start 96.2619 113.1666) (end 93.7066 115.7219) (width 0.2) (layer "B.Cu") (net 17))
 (segment (start 93.7066 115.7219) (end 93.7066 132.7247) (width 0.2) (layer "B.Cu") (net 17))
 (segment (start 99.49 114.72) (end 97.9366 113.1666) (width 0.2) (layer "B.Cu") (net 17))
 (segment (start 93.8714 144.6616) (end 92.1525 146.3805) (width 0.2) (layer "B.Cu") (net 17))
 (segment (start 93.7066 132.7247) (end 93.8714 132.8895) (width 0.2) (layer "B.Cu") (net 17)))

